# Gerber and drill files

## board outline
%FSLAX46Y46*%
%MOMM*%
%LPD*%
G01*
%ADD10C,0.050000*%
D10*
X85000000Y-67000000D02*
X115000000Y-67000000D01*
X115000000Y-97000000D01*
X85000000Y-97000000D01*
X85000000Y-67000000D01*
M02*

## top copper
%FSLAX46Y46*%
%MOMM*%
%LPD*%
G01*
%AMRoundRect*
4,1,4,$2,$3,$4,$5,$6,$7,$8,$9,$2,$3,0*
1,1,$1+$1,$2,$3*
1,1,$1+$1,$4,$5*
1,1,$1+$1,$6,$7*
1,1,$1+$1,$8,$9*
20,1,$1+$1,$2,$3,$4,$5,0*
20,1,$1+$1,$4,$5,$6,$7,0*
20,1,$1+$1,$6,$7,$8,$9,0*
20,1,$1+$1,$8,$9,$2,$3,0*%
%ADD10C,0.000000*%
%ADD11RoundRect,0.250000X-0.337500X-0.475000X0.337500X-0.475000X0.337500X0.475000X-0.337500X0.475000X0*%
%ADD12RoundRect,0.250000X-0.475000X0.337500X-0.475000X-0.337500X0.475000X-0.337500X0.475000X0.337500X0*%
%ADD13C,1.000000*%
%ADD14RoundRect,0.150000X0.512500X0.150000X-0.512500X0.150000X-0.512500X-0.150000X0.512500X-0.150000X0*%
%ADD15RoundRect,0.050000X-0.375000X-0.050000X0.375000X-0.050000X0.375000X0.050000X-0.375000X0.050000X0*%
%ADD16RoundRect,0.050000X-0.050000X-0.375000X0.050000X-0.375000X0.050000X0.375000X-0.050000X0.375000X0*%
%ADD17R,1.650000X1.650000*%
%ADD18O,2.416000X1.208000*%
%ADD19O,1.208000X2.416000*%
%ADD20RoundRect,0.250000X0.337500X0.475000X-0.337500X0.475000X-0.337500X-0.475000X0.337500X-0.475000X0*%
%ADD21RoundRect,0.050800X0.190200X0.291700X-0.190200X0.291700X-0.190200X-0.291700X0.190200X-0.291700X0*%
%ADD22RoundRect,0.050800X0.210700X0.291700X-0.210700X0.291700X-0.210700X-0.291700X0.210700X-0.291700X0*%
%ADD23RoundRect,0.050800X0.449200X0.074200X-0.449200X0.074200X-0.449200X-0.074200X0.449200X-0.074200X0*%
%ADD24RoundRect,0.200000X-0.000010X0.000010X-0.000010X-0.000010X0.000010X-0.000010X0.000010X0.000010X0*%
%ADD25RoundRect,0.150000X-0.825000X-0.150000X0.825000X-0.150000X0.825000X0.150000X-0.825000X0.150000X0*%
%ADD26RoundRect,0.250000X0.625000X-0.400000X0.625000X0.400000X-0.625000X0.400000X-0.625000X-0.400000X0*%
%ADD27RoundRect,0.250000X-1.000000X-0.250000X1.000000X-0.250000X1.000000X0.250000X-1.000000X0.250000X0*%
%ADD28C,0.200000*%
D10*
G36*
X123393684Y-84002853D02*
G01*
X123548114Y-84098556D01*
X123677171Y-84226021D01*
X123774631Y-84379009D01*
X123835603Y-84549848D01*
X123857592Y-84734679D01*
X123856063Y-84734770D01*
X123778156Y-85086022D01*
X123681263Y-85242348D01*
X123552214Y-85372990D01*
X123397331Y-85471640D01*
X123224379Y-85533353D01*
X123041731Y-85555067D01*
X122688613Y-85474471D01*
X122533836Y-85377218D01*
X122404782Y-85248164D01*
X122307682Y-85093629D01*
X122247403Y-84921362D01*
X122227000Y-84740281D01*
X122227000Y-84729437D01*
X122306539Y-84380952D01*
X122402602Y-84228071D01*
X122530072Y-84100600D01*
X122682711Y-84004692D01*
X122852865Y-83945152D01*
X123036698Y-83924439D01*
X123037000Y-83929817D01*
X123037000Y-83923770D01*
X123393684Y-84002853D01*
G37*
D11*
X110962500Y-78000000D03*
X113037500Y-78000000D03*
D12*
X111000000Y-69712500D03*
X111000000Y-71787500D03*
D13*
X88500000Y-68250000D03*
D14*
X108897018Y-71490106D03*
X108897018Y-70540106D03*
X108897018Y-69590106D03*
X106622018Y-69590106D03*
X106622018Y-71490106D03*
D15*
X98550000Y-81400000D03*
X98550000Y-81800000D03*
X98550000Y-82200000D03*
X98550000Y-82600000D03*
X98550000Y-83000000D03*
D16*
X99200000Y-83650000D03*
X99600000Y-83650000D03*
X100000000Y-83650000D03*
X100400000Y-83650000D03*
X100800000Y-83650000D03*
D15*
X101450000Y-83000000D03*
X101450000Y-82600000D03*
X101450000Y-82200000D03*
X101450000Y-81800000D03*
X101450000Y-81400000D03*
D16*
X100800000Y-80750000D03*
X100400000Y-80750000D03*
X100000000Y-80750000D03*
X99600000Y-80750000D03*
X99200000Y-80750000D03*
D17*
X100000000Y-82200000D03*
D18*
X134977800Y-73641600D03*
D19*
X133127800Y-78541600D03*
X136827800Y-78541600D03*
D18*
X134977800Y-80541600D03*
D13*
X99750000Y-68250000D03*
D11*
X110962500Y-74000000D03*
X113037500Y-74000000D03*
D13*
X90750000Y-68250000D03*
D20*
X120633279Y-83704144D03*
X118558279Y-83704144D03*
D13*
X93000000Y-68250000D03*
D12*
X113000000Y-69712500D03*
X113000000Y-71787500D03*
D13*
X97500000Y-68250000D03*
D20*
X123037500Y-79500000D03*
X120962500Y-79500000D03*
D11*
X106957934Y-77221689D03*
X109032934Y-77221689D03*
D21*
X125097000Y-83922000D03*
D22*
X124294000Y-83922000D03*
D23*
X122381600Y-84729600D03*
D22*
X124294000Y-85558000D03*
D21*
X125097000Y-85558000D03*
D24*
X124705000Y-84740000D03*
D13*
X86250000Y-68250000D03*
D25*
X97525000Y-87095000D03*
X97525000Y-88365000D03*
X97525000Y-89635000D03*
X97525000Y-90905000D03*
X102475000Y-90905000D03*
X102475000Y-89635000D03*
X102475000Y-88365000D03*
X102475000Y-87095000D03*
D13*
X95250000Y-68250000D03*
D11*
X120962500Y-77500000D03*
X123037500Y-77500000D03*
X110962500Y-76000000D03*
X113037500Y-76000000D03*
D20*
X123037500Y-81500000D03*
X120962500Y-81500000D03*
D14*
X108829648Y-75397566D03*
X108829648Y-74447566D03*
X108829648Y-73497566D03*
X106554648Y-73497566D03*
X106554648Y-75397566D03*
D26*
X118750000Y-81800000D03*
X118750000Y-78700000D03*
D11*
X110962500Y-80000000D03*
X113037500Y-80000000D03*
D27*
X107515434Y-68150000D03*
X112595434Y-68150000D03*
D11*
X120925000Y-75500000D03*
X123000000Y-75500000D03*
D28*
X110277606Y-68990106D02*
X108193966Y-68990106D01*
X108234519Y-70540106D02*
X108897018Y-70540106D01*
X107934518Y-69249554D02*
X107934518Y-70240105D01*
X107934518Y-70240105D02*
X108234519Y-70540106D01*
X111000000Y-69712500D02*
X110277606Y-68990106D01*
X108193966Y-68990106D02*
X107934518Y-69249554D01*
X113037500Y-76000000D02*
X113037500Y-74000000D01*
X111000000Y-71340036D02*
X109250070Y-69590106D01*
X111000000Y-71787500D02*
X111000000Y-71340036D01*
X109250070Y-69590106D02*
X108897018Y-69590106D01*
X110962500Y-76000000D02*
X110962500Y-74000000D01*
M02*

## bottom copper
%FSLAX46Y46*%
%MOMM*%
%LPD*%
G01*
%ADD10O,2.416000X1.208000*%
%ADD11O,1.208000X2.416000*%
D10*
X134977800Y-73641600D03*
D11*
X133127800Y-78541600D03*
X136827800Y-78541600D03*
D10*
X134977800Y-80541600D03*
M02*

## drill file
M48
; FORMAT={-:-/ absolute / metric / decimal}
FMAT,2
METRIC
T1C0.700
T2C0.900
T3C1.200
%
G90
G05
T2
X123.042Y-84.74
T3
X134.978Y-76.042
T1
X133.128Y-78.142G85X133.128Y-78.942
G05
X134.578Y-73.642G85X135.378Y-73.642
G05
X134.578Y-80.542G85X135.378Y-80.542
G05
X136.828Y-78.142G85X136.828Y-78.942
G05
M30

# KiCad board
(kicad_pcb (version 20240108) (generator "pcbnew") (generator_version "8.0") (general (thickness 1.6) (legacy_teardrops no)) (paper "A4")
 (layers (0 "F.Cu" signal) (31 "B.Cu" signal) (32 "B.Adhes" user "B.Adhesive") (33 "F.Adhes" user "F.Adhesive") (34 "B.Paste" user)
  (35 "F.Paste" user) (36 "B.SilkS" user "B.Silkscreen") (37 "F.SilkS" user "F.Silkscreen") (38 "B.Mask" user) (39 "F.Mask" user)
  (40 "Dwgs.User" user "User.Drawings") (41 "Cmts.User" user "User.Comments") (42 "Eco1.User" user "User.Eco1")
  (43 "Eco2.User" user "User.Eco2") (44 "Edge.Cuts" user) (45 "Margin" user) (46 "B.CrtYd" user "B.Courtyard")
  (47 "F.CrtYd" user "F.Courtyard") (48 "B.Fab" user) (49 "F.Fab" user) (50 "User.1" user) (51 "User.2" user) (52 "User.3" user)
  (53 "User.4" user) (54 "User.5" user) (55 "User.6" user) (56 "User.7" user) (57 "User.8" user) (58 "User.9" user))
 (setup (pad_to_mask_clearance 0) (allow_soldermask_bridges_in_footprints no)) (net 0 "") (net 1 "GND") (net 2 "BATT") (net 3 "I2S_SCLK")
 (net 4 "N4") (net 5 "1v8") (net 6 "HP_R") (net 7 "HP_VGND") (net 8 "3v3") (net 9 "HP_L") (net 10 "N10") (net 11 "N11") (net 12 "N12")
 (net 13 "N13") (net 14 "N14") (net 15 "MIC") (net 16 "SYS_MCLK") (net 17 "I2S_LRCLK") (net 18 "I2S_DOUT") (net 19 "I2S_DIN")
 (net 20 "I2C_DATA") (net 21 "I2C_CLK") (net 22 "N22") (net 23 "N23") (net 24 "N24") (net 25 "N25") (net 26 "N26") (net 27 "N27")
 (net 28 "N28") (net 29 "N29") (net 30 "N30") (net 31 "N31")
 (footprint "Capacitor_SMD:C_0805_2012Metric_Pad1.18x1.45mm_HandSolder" (layer "F.Cu") (at 112 78)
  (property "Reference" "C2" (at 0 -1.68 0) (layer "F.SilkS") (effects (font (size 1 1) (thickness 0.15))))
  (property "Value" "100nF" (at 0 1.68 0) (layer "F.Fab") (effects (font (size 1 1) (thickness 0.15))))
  (pad "1" smd roundrect (at -1.0375 0) (size 1.175 1.45) (layers "F.Cu" "F.Paste" "F.Mask") (roundrect_rratio 0.212766) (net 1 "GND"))
  (pad "2" smd roundrect (at 1.0375 0) (size 1.175 1.45) (layers "F.Cu" "F.Paste" "F.Mask") (roundrect_rratio 0.212766) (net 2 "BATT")))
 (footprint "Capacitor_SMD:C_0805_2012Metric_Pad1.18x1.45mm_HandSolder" (layer "F.Cu") (at 111 70.75 -90)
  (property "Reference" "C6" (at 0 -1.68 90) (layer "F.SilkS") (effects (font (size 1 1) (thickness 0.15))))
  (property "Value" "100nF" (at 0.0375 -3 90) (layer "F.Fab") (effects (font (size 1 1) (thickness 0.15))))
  (pad "1" smd roundrect (at -1.0375 0 270) (size 1.175 1.45) (layers "F.Cu" "F.Paste" "F.Mask") (roundrect_rratio 0.212766) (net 1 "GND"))
  (pad "2" smd roundrect (at 1.0375 0 270) (size 1.175 1.45) (layers "F.Cu" "F.Paste" "F.Mask") (roundrect_rratio 0.212766) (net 2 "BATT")))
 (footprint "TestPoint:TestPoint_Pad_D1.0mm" (layer "F.Cu") (at 88.5 68.25)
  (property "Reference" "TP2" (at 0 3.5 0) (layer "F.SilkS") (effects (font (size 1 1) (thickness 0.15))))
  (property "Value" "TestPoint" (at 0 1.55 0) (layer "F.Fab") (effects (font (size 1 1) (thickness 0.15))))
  (pad "1" smd circle (at 0 0) (size 1 1) (layers "F.Cu" "F.Mask") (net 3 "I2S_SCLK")))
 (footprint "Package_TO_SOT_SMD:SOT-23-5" (layer "F.Cu") (at 107.759518 70.540106 180)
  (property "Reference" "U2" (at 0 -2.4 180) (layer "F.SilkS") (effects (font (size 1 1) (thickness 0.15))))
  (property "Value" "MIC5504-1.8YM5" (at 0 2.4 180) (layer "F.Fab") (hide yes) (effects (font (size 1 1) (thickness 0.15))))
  (pad "1" smd roundrect (at -1.1375 -0.95 180) (size 1.325 0.6) (layers "F.Cu" "F.Paste" "F.Mask") (roundrect_rratio 0.25) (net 2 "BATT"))
  (pad "2" smd roundrect (at -1.1375 0 180) (size 1.325 0.6) (layers "F.Cu" "F.Paste" "F.Mask") (roundrect_rratio 0.25) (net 1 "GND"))
  (pad "3" smd roundrect (at -1.1375 0.95 180) (size 1.325 0.6) (layers "F.Cu" "F.Paste" "F.Mask") (roundrect_rratio 0.25) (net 2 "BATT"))
  (pad "4" smd roundrect (at 1.1375 0.95 180) (size 1.325 0.6) (layers "F.Cu" "F.Paste" "F.Mask") (roundrect_rratio 0.25) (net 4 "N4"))
  (pad "5" smd roundrect (at 1.1375 -0.95 180) (size 1.325 0.6) (layers "F.Cu" "F.Paste" "F.Mask") (roundrect_rratio 0.25) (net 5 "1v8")))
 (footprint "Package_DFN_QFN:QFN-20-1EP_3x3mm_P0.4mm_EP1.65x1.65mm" (layer "F.Cu") (at 100 82.2)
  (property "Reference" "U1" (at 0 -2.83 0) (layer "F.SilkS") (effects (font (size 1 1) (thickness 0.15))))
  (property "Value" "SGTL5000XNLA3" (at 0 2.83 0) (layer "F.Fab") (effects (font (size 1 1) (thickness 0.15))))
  (pad "" smd roundrect (at -0.41 -0.41) (size 0.67 0.67) (layers "F.Paste") (roundrect_rratio 0.25))
  (pad "" smd roundrect (at -0.41 0.41) (size 0.67 0.67) (layers "F.Paste") (roundrect_rratio 0.25))
  (pad "" smd roundrect (at 0.41 -0.41) (size 0.67 0.67) (layers "F.Paste") (roundrect_rratio 0.25))
  (pad "" smd roundrect (at 0.41 0.41) (size 0.67 0.67) (layers "F.Paste") (roundrect_rratio 0.25))
  (pad "1" smd roundrect (at -1.45 -0.8) (size 0.85 0.2) (layers "F.Cu" "F.Paste" "F.Mask") (roundrect_rratio 0.25) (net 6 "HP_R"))
  (pad "2" smd roundrect (at -1.45 -0.4) (size 0.85 0.2) (layers "F.Cu" "F.Paste" "F.Mask") (roundrect_rratio 0.25) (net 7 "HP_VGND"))
  (pad "3" smd roundrect (at -1.45 0) (size 0.85 0.2) (layers "F.Cu" "F.Paste" "F.Mask") (roundrect_rratio 0.25) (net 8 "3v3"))
  (pad "4" smd roundrect (at -1.45 0.4) (size 0.85 0.2) (layers "F.Cu" "F.Paste" "F.Mask") (roundrect_rratio 0.25) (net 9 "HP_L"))
  (pad "5" smd roundrect (at -1.45 0.8) (size 0.85 0.2) (layers "F.Cu" "F.Paste" "F.Mask") (roundrect_rratio 0.25) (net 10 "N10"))
  (pad "6" smd roundrect (at -0.8 1.45) (size 0.2 0.85) (layers "F.Cu" "F.Paste" "F.Mask") (roundrect_rratio 0.25) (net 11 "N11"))
  (pad "7" smd roundrect (at -0.4 1.45) (size 0.2 0.85) (layers "F.Cu" "F.Paste" "F.Mask") (roundrect_rratio 0.25) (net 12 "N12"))
  (pad "8" smd roundrect (at 0 1.45) (size 0.2 0.85) (layers "F.Cu" "F.Paste" "F.Mask") (roundrect_rratio 0.25) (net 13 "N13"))
  (pad "9" smd roundrect (at 0.4 1.45) (size 0.2 0.85) (layers "F.Cu" "F.Paste" "F.Mask") (roundrect_rratio 0.25) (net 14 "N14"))
  (pad "10" smd roundrect (at 0.8 1.45) (size 0.2 0.85) (layers "F.Cu" "F.Paste" "F.Mask") (roundrect_rratio 0.25) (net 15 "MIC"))
  (pad "11" smd roundrect (at 1.45 0.8) (size 0.85 0.2) (layers "F.Cu" "F.Paste" "F.Mask") (roundrect_rratio 0.25) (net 15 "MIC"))
  (pad "12" smd roundrect (at 1.45 0.4) (size 0.85 0.2) (layers "F.Cu" "F.Paste" "F.Mask") (roundrect_rratio 0.25) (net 8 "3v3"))
  (pad "13" smd roundrect (at 1.45 0) (size 0.85 0.2) (layers "F.Cu" "F.Paste" "F.Mask") (roundrect_rratio 0.25) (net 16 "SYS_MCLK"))
  (pad "14" smd roundrect (at 1.45 -0.4) (size 0.85 0.2) (layers "F.Cu" "F.Paste" "F.Mask") (roundrect_rratio 0.25) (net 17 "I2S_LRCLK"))
  (pad "15" smd roundrect (at 1.45 -0.8) (size 0.85 0.2) (layers "F.Cu" "F.Paste" "F.Mask") (roundrect_rratio 0.25) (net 3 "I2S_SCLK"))
  (pad "16" smd roundrect (at 0.8 -1.45) (size 0.2 0.85) (layers "F.Cu" "F.Paste" "F.Mask") (roundrect_rratio 0.25) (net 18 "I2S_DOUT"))
  (pad "17" smd roundrect (at 0.4 -1.45) (size 0.2 0.85) (layers "F.Cu" "F.Paste" "F.Mask") (roundrect_rratio 0.25) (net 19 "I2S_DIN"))
  (pad "18" smd roundrect (at 0 -1.45) (size 0.2 0.85) (layers "F.Cu" "F.Paste" "F.Mask") (roundrect_rratio 0.25) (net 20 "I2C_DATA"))
  (pad "19" smd roundrect (at -0.4 -1.45) (size 0.2 0.85) (layers "F.Cu" "F.Paste" "F.Mask") (roundrect_rratio 0.25) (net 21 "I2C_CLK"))
  (pad "20" smd roundrect (at -0.8 -1.45) (size 0.2 0.85) (layers "F.Cu" "F.Paste" "F.Mask") (roundrect_rratio 0.25) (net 5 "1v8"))
  (pad "21" smd rect (at 0 0) (size 1.65 1.65) (layers "F.Cu" "F.Mask") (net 1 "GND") (zone_connect 2)))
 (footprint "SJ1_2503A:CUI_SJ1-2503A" (layer "F.Cu") (at 134.9778 73.6416)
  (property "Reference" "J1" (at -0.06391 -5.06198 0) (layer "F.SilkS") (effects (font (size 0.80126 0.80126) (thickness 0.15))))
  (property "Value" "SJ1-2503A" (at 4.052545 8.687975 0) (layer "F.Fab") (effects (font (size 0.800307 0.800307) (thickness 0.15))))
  (pad "" np_thru_hole circle (at 0 2.4) (size 1.2 1.2) (drill 1.2) (layers "*.Cu" "*.Mask"))
  (pad "1" thru_hole oval (at 0 0) (size 2.416 1.208) (drill oval 1.5 0.7) (layers "*.Cu" "*.Mask") (remove_unused_layers no)
   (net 7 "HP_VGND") (solder_mask_margin 0.102))
  (pad "2" thru_hole oval (at -1.85 4.9) (size 1.208 2.416) (drill oval 0.7 1.5) (layers "*.Cu" "*.Mask") (remove_unused_layers no)
   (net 6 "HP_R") (solder_mask_margin 0.102))
  (pad "3" thru_hole oval (at 1.85 4.9) (size 1.208 2.416) (drill oval 0.7 1.5) (layers "*.Cu" "*.Mask") (remove_unused_layers no)
   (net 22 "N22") (solder_mask_margin 0.102))
  (pad "4" thru_hole oval (at 0 6.9) (size 2.416 1.208) (drill oval 1.5 0.7) (layers "*.Cu" "*.Mask") (remove_unused_layers no)
   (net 9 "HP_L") (solder_mask_margin 0.102)))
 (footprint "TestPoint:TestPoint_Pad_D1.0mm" (layer "F.Cu") (at 99.75 68.25)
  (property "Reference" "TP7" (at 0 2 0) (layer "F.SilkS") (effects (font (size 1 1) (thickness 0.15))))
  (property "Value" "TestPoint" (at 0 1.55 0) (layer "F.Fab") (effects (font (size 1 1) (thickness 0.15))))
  (pad "1" smd circle (at 0 0) (size 1 1) (layers "F.Cu" "F.Mask") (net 16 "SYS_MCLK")))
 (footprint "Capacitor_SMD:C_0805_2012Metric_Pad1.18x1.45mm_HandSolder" (layer "F.Cu") (at 112 74)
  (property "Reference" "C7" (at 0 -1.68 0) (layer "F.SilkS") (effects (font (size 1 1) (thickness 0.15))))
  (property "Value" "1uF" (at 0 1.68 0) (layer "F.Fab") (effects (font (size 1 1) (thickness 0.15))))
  (pad "1" smd roundrect (at -1.0375 0) (size 1.175 1.45) (layers "F.Cu" "F.Paste" "F.Mask") (roundrect_rratio 0.212766) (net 5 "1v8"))
  (pad "2" smd roundrect (at 1.0375 0) (size 1.175 1.45) (layers "F.Cu" "F.Paste" "F.Mask") (roundrect_rratio 0.212766) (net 1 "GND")))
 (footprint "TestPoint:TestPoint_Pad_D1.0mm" (layer "F.Cu") (at 90.75 68.25)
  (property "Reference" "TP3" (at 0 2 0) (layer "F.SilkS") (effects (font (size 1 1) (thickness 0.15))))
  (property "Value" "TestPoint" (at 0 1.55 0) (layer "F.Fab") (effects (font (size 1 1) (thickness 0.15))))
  (pad "1" smd circle (at 0 0) (size 1 1) (layers "F.Cu" "F.Mask") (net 18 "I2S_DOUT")))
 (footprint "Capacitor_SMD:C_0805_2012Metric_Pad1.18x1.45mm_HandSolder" (layer "F.Cu") (at 119.595779 83.704144 180)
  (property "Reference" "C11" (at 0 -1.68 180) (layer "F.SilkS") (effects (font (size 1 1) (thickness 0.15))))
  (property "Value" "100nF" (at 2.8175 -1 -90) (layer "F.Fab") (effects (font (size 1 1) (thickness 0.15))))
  (pad "1" smd roundrect (at -1.0375 0 180) (size 1.175 1.45) (layers "F.Cu" "F.Paste" "F.Mask") (roundrect_rratio 0.212766) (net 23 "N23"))
  (pad "2" smd roundrect (at 1.0375 0 180) (size 1.175 1.45) (layers "F.Cu" "F.Paste" "F.Mask") (roundrect_rratio 0.212766) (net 15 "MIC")))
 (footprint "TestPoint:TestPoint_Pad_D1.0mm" (layer "F.Cu") (at 93 68.25)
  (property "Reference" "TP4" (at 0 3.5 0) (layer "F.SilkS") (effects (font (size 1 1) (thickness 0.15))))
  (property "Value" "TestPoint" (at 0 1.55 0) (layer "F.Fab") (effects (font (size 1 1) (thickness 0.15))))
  (pad "1" smd circle (at 0 0) (size 1 1) (layers "F.Cu" "F.Mask") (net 19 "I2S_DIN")))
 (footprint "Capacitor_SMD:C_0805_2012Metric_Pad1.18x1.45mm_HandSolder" (layer "F.Cu") (at 113 70.75 -90)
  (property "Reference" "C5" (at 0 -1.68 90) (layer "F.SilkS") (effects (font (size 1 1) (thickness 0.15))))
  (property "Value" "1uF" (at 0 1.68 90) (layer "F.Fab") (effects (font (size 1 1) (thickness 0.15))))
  (pad "1" smd roundrect (at -1.0375 0 270) (size 1.175 1.45) (layers "F.Cu" "F.Paste" "F.Mask") (roundrect_rratio 0.212766) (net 1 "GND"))
  (pad "2" smd roundrect (at 1.0375 0 270) (size 1.175 1.45) (layers "F.Cu" "F.Paste" "F.Mask") (roundrect_rratio 0.212766) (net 2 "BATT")))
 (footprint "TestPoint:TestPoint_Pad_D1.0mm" (layer "F.Cu") (at 97.5 68.25)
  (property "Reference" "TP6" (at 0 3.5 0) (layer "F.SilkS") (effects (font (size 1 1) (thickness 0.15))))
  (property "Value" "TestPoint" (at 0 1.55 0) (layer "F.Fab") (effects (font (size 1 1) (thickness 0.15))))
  (pad "1" smd circle (at 0 0) (size 1 1) (layers "F.Cu" "F.Mask") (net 21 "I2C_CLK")))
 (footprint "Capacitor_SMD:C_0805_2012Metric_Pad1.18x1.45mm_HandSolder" (layer "F.Cu") (at 122 79.5 180)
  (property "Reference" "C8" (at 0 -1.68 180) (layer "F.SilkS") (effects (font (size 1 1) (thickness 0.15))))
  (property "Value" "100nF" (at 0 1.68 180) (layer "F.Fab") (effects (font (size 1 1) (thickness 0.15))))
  (pad "1" smd roundrect (at -1.0375 0 180) (size 1.175 1.45) (layers "F.Cu" "F.Paste" "F.Mask") (roundrect_rratio 0.212766) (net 8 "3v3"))
  (pad "2" smd roundrect (at 1.0375 0 180) (size 1.175 1.45) (layers "F.Cu" "F.Paste" "F.Mask") (roundrect_rratio 0.212766) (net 1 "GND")))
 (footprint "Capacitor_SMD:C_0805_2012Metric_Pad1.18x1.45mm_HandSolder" (layer "F.Cu") (at 107.995434 77.221689)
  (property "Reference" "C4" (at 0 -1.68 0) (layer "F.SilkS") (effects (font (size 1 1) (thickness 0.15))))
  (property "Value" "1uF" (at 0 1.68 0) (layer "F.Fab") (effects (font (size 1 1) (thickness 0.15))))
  (pad "1" smd roundrect (at -1.0375 0) (size 1.175 1.45) (layers "F.Cu" "F.Paste" "F.Mask") (roundrect_rratio 0.212766) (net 8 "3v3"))
  (pad "2" smd roundrect (at 1.0375 0) (size 1.175 1.45) (layers "F.Cu" "F.Paste" "F.Mask") (roundrect_rratio 0.212766) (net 1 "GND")))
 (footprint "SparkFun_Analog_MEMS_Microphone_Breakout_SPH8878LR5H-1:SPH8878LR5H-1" (layer "F.Cu") (at 123.042 84.74 -90)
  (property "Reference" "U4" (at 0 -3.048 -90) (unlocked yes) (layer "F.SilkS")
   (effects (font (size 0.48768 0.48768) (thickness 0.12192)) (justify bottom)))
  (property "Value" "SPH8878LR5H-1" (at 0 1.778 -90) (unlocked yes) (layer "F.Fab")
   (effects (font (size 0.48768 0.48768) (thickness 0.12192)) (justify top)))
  (fp_poly
   (pts (xy -0.00523 -0.814063) (xy 0.346022 -0.736156) (xy 0.502348 -0.639263) (xy 0.63299 -0.510214) (xy 0.73164 -0.355331)
    (xy 0.793353 -0.182379) (xy 0.815067 0.000269) (xy 0.734471 0.353387) (xy 0.637218 0.508164) (xy 0.508164 0.637218)
    (xy 0.353629 0.734318) (xy 0.181362 0.794597) (xy 0.000281 0.815) (xy -0.010563 0.815) (xy -0.359048 0.735461) (xy -0.511929 0.639398)
    (xy -0.6394 0.511928) (xy -0.735308 0.359289) (xy -0.794848 0.189135) (xy -0.815561 0.005302) (xy -0.810183 0.005) (xy -0.81623 0.005)
    (xy -0.737147 -0.351684) (xy -0.641444 -0.506114) (xy -0.513979 -0.635171) (xy -0.360991 -0.732631) (xy -0.190152 -0.793603)
    (xy -0.005321 -0.815592))
   (stroke (width 0) (type default)) (fill solid) (layer "F.Cu"))
  (pad "" np_thru_hole circle (at 0 0 270) (size 0.9 0.9) (drill 0.9) (layers "*.Cu" "*.Mask"))
  (pad "1" smd roundrect (at -0.818 -2.055 180) (size 0.482 0.685) (layers "F.Cu" "F.Paste" "F.Mask") (roundrect_rratio 0.1053941909)
   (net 23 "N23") (solder_mask_margin 0.0635) (thermal_bridge_angle 0))
  (pad "2" smd roundrect (at -0.818 -1.252 180) (size 0.523 0.685) (layers "F.Cu" "F.Paste" "F.Mask") (roundrect_rratio 0.09713193117)
   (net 1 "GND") (solder_mask_margin 0.0635) (thermal_bridge_angle 0))
  (pad "3" smd roundrect (at -0.0104 0.6604 180) (size 1 0.25) (layers "F.Cu") (roundrect_rratio 0.2032) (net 1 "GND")
   (solder_mask_margin 0.0635) (thermal_bridge_angle 0))
  (pad "4" smd roundrect (at 0.818 -1.252 180) (size 0.523 0.685) (layers "F.Cu" "F.Paste" "F.Mask") (roundrect_rratio 0.09713193117)
   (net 1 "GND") (solder_mask_margin 0.0635) (thermal_bridge_angle 0))
  (pad "5" smd roundrect (at 0.818 -2.055 180) (size 0.482 0.685) (layers "F.Cu" "F.Paste" "F.Mask") (roundrect_rratio 0.1053941909)
   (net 8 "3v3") (solder_mask_margin 0.0635) (thermal_bridge_angle 0))
  (pad "6" smd roundrect (at 0 -1.663 270) (size 0.4 0.4) (layers "F.Cu" "F.Paste" "F.Mask") (roundrect_rratio 0.5) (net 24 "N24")
   (solder_mask_margin 0.0635) (thermal_bridge_angle 0)))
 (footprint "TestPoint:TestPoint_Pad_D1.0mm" (layer "F.Cu") (at 86.25 68.25)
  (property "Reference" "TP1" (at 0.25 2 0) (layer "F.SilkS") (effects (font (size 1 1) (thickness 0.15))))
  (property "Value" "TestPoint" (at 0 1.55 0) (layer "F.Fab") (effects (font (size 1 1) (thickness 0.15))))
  (pad "1" smd circle (at 0 0) (size 1 1) (layers "F.Cu" "F.Mask") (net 17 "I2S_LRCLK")))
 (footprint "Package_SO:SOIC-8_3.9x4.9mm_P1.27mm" (layer "F.Cu") (at 100 89)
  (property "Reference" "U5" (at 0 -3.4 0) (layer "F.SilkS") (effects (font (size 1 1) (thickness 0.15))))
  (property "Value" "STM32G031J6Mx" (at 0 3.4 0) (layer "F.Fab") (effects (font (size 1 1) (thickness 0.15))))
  (pad "1" smd roundrect (at -2.475 -1.905) (size 1.95 0.6) (layers "F.Cu" "F.Paste" "F.Mask") (roundrect_rratio 0.25) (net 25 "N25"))
  (pad "2" smd roundrect (at -2.475 -0.635) (size 1.95 0.6) (layers "F.Cu" "F.Paste" "F.Mask") (roundrect_rratio 0.25) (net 8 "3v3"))
  (pad "3" smd roundrect (at -2.475 0.635) (size 1.95 0.6) (layers "F.Cu" "F.Paste" "F.Mask") (roundrect_rratio 0.25) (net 1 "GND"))
  (pad "4" smd roundrect (at -2.475 1.905) (size 1.95 0.6) (layers "F.Cu" "F.Paste" "F.Mask") (roundrect_rratio 0.25) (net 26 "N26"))
  (pad "5" smd roundrect (at 2.475 1.905) (size 1.95 0.6) (layers "F.Cu" "F.Paste" "F.Mask") (roundrect_rratio 0.25) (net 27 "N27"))
  (pad "6" smd roundrect (at 2.475 0.635) (size 1.95 0.6) (layers "F.Cu" "F.Paste" "F.Mask") (roundrect_rratio 0.25) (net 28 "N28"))
  (pad "7" smd roundrect (at 2.475 -0.635) (size 1.95 0.6) (layers "F.Cu" "F.Paste" "F.Mask") (roundrect_rratio 0.25) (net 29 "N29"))
  (pad "8" smd roundrect (at 2.475 -1.905) (size 1.95 0.6) (layers "F.Cu" "F.Paste" "F.Mask") (roundrect_rratio 0.25) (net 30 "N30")))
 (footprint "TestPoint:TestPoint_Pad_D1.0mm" (layer "F.Cu") (at 95.25 68.25)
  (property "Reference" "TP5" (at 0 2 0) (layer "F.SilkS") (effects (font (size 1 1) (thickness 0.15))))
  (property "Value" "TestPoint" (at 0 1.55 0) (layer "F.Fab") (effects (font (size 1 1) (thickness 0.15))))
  (pad "1" smd circle (at 0 0) (size 1 1) (layers "F.Cu" "F.Mask") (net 20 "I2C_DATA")))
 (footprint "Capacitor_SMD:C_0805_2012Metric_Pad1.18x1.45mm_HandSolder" (layer "F.Cu") (at 122 77.5)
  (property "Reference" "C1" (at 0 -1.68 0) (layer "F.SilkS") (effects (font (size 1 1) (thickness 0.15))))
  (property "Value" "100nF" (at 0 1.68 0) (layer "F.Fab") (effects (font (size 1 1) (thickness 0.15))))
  (pad "1" smd roundrect (at -1.0375 0) (size 1.175 1.45) (layers "F.Cu" "F.Paste" "F.Mask") (roundrect_rratio 0.212766) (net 1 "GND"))
  (pad "2" smd roundrect (at 1.0375 0) (size 1.175 1.45) (layers "F.Cu" "F.Paste" "F.Mask") (roundrect_rratio 0.212766) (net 10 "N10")))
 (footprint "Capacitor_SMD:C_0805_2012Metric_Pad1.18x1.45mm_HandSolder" (layer "F.Cu") (at 112 76)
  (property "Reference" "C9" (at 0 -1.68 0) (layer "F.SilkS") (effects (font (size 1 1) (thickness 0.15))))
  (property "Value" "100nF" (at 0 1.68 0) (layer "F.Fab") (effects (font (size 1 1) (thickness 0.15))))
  (pad "1" smd roundrect (at -1.0375 0) (size 1.175 1.45) (layers "F.Cu" "F.Paste" "F.Mask") (roundrect_rratio 0.212766) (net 5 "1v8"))
  (pad "2" smd roundrect (at 1.0375 0) (size 1.175 1.45) (layers "F.Cu" "F.Paste" "F.Mask") (roundrect_rratio 0.212766) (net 1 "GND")))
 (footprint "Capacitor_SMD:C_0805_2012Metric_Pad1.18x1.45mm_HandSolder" (layer "F.Cu") (at 122 81.5 180)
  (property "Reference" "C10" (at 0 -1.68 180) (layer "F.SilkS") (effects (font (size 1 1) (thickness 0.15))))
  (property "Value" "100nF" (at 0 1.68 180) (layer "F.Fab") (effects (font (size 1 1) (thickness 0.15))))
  (pad "1" smd roundrect (at -1.0375 0 180) (size 1.175 1.45) (layers "F.Cu" "F.Paste" "F.Mask") (roundrect_rratio 0.212766) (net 8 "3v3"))
  (pad "2" smd roundrect (at 1.0375 0 180) (size 1.175 1.45) (layers "F.Cu" "F.Paste" "F.Mask") (roundrect_rratio 0.212766) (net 1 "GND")))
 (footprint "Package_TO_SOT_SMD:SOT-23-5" (layer "F.Cu") (at 107.692148 74.447566 180)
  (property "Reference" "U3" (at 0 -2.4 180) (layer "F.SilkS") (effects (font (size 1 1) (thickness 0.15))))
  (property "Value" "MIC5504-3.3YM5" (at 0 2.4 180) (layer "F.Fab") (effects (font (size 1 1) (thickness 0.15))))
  (pad "1" smd roundrect (at -1.1375 -0.95 180) (size 1.325 0.6) (layers "F.Cu" "F.Paste" "F.Mask") (roundrect_rratio 0.25) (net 2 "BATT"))
  (pad "2" smd roundrect (at -1.1375 0 180) (size 1.325 0.6) (layers "F.Cu" "F.Paste" "F.Mask") (roundrect_rratio 0.25) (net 1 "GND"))
  (pad "3" smd roundrect (at -1.1375 0.95 180) (size 1.325 0.6) (layers "F.Cu" "F.Paste" "F.Mask") (roundrect_rratio 0.25) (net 2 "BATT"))
  (pad "4" smd roundrect (at 1.1375 0.95 180) (size 1.325 0.6) (layers "F.Cu" "F.Paste" "F.Mask") (roundrect_rratio 0.25) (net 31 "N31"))
  (pad "5" smd roundrect (at 1.1375 -0.95 180) (size 1.325 0.6) (layers "F.Cu" "F.Paste" "F.Mask") (roundrect_rratio 0.25) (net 8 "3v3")))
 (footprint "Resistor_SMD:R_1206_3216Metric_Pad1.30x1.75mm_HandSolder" (layer "F.Cu") (at 118.75 80.25 90)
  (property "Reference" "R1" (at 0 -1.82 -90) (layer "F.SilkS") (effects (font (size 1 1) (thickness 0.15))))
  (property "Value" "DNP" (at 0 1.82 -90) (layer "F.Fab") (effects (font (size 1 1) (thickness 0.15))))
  (pad "1" smd roundrect (at -1.55 0 90) (size 1.3 1.75) (layers "F.Cu" "F.Paste" "F.Mask") (roundrect_rratio 0.192308) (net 15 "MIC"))
  (pad "2" smd roundrect (at 1.55 0 90) (size 1.3 1.75) (layers "F.Cu" "F.Paste" "F.Mask") (roundrect_rratio 0.192308) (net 15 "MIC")))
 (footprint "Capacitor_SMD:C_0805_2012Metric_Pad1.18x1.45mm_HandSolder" (layer "F.Cu") (at 112 80)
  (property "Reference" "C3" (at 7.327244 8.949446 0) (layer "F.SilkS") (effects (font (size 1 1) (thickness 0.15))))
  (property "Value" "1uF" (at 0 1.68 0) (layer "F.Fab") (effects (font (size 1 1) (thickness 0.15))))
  (pad "1" smd roundrect (at -1.0375 0) (size 1.175 1.45) (layers "F.Cu" "F.Paste" "F.Mask") (roundrect_rratio 0.212766) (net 1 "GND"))
  (pad "2" smd roundrect (at 1.0375 0) (size 1.175 1.45) (layers "F.Cu" "F.Paste" "F.Mask") (roundrect_rratio 0.212766) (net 2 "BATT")))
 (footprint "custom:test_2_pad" (layer "F.Cu") (at 110.055434 63.07)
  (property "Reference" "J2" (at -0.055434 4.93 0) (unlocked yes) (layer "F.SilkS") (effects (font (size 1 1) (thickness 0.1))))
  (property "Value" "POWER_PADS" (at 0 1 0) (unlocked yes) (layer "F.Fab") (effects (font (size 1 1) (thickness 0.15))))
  (pad "1" smd roundrect (at -2.54 5.08) (size 2.5 1) (layers "F.Cu" "F.Paste" "F.Mask") (roundrect_rratio 0.25) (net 2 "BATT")
   (thermal_bridge_angle 45))
  (pad "2" smd roundrect (at 2.54 5.08) (size 2.5 1) (layers "F.Cu" "F.Paste" "F.Mask") (roundrect_rratio 0.25) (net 1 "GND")
   (thermal_bridge_angle 45)))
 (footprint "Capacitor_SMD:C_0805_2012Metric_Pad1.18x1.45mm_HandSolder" (layer "F.Cu") (at 121.9625 75.5)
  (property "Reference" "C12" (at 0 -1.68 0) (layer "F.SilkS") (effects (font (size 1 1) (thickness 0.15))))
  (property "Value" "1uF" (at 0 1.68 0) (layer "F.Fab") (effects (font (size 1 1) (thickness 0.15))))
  (pad "1" smd roundrect (at -1.0375 0) (size 1.175 1.45) (layers "F.Cu" "F.Paste" "F.Mask") (roundrect_rratio 0.212766) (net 1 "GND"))
  (pad "2" smd roundrect (at 1.0375 0) (size 1.175 1.45) (layers "F.Cu" "F.Paste" "F.Mask") (roundrect_rratio 0.212766) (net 8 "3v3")))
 (gr_rect (start 85 67) (end 115 97) (stroke (width 0.05) (type default)) (fill none) (layer "Edge.Cuts"))
 (segment (start 110.277606 68.990106) (end 108.193966 68.990106) (width 0.2) (layer "F.Cu") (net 1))
 (segment (start 108.234519 70.540106) (end 108.897018 70.540106) (width 0.2) (layer "F.Cu") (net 1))
 (segment (start 107.934518 69.249554) (end 107.934518 70.240105) (width 0.2) (layer "F.Cu") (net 1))
 (segment (start 107.934518 70.240105) (end 108.234519 70.540106) (width 0.2) (layer "F.Cu") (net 1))
 (segment (start 111 69.7125) (end 110.277606 68.990106) (width 0.2) (layer "F.Cu") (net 1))
 (segment (start 108.193966 68.990106) (end 107.934518 69.249554) (width 0.2) (layer "F.Cu") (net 1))
 (segment (start 113.0375 76) (end 113.0375 74) (width 0.2) (layer "F.Cu") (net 1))
 (segment (start 111 71.340036) (end 109.25007 69.590106) (width 0.2) (layer "F.Cu") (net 2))
 (segment (start 111 71.7875) (end 111 71.340036) (width 0.2) (layer "F.Cu") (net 2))
 (segment (start 109.25007 69.590106) (end 108.897018 69.590106) (width 0.2) (layer "F.Cu") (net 2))
 (segment (start 110.9625 76) (end 110.9625 74) (width 0.2) (layer "F.Cu") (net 5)))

